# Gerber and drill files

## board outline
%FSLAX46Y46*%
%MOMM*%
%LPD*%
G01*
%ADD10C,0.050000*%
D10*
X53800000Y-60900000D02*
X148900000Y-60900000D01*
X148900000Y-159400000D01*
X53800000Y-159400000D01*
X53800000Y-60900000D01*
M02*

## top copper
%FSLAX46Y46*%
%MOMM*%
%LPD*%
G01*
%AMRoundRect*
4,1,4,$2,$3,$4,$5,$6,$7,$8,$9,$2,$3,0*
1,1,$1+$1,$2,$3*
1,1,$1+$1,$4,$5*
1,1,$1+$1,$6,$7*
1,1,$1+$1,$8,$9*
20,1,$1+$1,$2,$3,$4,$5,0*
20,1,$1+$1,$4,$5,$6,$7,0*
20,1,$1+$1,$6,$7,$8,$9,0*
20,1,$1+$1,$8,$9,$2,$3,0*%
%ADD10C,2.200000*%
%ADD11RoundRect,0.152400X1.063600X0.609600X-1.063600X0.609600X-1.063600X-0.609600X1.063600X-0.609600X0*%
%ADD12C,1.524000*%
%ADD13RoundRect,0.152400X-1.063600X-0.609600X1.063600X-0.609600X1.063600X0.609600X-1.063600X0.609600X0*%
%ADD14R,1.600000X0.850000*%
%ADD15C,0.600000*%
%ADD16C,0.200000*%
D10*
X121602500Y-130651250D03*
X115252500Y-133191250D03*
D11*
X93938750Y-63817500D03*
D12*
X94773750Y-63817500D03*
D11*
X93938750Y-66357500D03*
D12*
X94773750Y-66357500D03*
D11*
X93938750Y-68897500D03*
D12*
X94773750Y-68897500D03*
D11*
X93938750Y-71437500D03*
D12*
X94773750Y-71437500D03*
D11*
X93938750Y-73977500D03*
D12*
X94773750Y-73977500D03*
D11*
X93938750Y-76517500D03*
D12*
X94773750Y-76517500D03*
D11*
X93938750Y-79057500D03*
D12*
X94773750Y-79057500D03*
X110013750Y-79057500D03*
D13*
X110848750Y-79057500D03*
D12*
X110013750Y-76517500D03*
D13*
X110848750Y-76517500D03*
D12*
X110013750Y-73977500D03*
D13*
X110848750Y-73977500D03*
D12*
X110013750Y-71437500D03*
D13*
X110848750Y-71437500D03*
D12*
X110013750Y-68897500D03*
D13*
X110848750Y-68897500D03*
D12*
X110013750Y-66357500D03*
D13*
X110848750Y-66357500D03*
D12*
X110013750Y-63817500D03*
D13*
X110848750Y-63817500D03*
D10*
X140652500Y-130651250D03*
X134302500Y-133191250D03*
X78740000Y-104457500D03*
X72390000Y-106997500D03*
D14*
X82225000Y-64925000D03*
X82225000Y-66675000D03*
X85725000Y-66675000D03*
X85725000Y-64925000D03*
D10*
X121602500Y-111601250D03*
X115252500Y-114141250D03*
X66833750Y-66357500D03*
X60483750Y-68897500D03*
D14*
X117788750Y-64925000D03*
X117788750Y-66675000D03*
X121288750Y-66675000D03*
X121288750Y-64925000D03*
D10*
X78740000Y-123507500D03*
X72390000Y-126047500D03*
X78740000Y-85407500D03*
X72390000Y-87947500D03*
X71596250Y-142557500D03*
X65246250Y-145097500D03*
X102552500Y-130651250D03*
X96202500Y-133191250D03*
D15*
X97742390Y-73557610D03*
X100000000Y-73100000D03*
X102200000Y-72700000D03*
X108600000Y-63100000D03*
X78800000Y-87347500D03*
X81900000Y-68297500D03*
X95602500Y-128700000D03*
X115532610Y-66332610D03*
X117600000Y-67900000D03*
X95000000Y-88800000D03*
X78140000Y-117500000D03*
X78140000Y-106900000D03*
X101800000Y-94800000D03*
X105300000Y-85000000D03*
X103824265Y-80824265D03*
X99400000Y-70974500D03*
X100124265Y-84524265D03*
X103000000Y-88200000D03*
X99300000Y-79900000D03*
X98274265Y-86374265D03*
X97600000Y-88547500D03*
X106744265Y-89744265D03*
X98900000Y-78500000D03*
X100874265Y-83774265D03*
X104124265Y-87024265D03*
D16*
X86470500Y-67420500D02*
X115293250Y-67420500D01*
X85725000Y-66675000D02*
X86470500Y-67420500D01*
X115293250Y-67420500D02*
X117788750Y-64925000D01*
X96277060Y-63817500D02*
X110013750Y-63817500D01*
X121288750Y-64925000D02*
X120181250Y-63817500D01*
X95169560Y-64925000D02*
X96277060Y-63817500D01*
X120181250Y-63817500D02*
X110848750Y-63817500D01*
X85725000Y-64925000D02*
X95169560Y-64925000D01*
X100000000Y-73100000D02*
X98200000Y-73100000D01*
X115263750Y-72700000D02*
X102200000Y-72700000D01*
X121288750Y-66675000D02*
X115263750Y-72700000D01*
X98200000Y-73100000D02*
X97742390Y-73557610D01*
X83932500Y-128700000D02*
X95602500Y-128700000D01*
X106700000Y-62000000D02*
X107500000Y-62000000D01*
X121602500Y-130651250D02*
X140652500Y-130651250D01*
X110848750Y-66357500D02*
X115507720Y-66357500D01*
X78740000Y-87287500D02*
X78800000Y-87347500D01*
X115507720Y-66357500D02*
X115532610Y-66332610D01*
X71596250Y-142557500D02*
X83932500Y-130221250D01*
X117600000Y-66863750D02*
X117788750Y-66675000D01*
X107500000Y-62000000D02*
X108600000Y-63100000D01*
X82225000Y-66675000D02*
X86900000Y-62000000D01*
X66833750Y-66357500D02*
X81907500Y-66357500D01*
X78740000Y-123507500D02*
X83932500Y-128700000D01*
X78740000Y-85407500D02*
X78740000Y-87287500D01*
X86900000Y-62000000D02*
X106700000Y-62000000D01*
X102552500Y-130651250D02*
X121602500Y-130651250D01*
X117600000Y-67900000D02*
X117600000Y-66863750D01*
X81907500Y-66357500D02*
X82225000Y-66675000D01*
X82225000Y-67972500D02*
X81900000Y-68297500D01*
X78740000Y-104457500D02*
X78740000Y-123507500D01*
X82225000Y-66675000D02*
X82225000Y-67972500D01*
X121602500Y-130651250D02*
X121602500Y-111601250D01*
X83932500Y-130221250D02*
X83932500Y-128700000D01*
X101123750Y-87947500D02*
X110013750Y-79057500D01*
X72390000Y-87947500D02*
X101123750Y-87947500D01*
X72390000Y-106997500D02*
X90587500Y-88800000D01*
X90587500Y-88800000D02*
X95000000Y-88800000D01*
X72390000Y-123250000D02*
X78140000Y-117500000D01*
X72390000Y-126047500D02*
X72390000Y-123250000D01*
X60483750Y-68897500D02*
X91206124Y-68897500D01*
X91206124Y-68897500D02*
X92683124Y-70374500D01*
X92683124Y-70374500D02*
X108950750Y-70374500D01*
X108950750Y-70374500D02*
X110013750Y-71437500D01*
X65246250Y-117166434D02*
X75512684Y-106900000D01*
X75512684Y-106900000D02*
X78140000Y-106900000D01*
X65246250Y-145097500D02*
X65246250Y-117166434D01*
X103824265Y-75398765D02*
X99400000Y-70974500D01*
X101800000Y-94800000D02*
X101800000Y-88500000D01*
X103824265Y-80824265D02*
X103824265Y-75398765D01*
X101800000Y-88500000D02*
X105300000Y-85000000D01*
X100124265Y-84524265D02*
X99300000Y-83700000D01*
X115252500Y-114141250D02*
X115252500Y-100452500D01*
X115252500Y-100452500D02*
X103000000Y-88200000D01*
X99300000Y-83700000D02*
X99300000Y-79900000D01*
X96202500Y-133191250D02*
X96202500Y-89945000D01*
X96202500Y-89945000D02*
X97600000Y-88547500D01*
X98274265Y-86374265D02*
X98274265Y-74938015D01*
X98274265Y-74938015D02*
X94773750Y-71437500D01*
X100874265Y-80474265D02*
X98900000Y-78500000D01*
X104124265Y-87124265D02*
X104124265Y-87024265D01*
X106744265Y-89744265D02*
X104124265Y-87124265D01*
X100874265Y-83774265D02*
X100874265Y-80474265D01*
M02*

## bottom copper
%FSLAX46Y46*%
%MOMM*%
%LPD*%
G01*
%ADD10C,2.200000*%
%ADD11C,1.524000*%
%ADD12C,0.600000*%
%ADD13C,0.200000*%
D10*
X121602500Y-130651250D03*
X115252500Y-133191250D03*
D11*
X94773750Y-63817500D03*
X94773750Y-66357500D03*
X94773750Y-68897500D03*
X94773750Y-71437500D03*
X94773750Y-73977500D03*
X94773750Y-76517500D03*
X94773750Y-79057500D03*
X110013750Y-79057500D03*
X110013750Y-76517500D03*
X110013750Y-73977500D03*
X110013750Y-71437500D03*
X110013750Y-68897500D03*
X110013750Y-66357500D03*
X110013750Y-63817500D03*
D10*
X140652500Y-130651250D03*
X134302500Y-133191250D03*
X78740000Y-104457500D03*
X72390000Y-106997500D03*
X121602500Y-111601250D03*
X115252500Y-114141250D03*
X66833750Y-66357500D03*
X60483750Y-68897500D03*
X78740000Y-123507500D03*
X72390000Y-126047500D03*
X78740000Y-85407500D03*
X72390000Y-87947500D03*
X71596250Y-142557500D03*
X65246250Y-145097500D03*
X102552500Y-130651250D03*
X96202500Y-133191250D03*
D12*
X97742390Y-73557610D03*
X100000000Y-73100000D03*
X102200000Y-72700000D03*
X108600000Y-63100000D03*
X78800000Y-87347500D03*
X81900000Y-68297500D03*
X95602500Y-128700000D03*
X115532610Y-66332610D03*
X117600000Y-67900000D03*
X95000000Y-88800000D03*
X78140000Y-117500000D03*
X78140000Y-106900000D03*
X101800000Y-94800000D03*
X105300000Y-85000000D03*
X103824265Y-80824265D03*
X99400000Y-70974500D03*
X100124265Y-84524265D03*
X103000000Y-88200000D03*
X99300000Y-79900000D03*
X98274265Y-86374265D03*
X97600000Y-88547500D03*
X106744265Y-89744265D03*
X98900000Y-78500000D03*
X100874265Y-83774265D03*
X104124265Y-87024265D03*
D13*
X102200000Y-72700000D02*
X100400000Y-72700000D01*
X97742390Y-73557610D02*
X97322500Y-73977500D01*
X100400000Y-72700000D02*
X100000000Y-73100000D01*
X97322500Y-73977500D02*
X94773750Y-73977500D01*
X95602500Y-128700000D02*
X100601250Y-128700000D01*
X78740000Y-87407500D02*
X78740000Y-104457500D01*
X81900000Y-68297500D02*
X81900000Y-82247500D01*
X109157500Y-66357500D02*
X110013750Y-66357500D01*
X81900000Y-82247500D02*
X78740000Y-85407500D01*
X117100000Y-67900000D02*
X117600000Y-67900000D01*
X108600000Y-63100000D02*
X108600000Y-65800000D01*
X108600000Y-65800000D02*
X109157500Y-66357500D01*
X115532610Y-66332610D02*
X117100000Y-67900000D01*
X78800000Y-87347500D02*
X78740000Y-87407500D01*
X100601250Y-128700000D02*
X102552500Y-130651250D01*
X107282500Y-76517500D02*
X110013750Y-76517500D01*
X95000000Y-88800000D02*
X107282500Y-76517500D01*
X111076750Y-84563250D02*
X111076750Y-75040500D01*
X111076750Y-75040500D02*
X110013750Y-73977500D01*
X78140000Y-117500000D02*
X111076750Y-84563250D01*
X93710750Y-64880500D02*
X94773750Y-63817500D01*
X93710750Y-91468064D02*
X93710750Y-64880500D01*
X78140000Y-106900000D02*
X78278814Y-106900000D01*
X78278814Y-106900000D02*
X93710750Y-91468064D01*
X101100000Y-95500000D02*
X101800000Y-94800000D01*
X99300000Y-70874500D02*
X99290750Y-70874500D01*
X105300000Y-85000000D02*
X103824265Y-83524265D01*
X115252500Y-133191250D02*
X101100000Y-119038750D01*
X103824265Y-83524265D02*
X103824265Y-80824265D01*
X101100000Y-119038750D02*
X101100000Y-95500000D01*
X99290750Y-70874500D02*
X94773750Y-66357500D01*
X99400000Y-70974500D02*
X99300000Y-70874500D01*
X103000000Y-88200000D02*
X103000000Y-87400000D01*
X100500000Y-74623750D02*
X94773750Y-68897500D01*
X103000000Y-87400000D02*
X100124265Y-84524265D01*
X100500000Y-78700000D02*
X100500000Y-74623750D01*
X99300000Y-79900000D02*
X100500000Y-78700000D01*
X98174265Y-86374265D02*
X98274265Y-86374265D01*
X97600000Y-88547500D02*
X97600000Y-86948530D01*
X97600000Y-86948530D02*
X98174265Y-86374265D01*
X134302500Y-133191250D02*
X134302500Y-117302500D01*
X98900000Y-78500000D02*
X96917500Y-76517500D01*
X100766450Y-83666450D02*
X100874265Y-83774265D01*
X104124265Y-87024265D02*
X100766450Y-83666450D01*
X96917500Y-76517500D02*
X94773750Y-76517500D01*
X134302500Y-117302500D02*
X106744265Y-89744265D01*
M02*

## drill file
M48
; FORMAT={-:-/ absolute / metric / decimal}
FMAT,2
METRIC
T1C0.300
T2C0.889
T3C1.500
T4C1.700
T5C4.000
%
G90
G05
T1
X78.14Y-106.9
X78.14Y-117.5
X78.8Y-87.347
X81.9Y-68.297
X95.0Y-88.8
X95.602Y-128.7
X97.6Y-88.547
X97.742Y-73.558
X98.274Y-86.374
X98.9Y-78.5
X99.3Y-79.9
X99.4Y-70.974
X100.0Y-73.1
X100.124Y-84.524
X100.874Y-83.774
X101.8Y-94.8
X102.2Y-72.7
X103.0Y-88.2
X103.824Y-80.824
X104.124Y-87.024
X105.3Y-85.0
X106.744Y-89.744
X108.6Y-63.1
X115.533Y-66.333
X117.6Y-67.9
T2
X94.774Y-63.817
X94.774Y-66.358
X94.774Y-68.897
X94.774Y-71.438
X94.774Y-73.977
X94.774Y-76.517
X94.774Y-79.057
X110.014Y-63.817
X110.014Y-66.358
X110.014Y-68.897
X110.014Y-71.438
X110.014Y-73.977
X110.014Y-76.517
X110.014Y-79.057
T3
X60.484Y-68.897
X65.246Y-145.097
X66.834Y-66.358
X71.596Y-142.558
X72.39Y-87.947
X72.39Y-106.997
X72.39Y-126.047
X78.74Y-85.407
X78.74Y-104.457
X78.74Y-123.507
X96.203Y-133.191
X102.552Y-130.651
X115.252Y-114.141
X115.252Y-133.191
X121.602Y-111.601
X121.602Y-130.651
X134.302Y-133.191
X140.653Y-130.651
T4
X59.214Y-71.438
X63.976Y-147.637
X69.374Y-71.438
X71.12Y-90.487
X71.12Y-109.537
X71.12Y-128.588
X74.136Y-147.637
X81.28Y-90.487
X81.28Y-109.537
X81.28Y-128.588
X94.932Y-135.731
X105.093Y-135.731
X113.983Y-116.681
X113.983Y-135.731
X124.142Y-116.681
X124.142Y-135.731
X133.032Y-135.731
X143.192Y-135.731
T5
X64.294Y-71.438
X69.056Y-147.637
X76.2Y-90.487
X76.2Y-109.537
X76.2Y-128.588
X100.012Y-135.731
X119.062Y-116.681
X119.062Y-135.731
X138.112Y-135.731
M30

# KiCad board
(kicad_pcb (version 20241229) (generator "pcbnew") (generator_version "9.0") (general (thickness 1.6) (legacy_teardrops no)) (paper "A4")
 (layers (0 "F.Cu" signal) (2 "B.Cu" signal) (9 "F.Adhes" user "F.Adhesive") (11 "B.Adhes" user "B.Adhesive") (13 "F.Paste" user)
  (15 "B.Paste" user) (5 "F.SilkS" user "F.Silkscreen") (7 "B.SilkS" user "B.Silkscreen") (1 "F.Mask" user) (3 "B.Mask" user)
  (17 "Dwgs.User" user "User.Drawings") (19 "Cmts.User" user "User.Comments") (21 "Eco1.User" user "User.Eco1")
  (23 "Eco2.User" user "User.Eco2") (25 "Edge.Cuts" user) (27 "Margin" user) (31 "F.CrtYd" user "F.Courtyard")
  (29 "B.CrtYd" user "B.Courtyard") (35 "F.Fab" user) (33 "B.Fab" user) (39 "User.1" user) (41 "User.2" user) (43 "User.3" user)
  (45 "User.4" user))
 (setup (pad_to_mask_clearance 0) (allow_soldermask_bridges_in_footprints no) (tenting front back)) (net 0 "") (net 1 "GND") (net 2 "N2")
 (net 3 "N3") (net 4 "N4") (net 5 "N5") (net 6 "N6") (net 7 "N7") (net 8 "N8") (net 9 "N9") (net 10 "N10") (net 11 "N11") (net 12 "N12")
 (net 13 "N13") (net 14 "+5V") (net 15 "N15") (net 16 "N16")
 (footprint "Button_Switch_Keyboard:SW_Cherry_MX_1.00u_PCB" (layer "F.Cu") (at 121.6025 130.65125)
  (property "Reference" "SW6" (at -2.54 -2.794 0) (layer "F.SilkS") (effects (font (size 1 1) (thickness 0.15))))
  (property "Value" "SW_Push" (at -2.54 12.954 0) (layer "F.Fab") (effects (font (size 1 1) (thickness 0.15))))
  (pad "" np_thru_hole circle (at -7.62 5.08) (size 1.7 1.7) (drill 1.7) (layers "*.Cu" "*.Mask"))
  (pad "" np_thru_hole circle (at -2.54 5.08) (size 4 4) (drill 4) (layers "*.Cu" "*.Mask"))
  (pad "" np_thru_hole circle (at 2.54 5.08) (size 1.7 1.7) (drill 1.7) (layers "*.Cu" "*.Mask"))
  (pad "1" thru_hole circle (at 0 0) (size 2.2 2.2) (drill 1.5) (layers "*.Cu" "*.Mask") (remove_unused_layers no) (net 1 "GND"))
  (pad "2" thru_hole circle (at -6.35 2.54) (size 2.2 2.2) (drill 1.5) (layers "*.Cu" "*.Mask") (remove_unused_layers no) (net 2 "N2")))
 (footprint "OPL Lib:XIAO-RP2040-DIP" (layer "F.Cu") (at 102.39375 71.4375)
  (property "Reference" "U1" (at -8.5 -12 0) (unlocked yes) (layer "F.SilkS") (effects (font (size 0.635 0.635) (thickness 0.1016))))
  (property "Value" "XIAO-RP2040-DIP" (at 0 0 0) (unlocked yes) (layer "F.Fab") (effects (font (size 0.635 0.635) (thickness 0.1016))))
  (pad "1" smd roundrect (at -8.455 -7.62 180) (size 2.432 1.524) (layers "F.Cu" "F.Mask") (roundrect_rratio 0.1) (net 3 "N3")
   (thermal_bridge_angle 45))
  (pad "1" thru_hole circle (at -7.62 -7.62 180) (size 1.524 1.524) (drill 0.889) (layers "*.Cu" "*.Mask") (remove_unused_layers no)
   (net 3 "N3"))
  (pad "2" smd roundrect (at -8.455 -5.08 180) (size 2.432 1.524) (layers "F.Cu" "F.Mask") (roundrect_rratio 0.1) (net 2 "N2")
   (thermal_bridge_angle 45))
  (pad "2" thru_hole circle (at -7.62 -5.08 180) (size 1.524 1.524) (drill 0.889) (layers "*.Cu" "*.Mask") (remove_unused_layers no)
   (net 2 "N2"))
  (pad "3" smd roundrect (at -8.455 -2.54 180) (size 2.432 1.524) (layers "F.Cu" "F.Mask") (roundrect_rratio 0.1) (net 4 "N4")
   (thermal_bridge_angle 45))
  (pad "3" thru_hole circle (at -7.62 -2.54 180) (size 1.524 1.524) (drill 0.889) (layers "*.Cu" "*.Mask") (remove_unused_layers no)
   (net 4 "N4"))
  (pad "4" smd roundrect (at -8.455 0 180) (size 2.432 1.524) (layers "F.Cu" "F.Mask") (roundrect_rratio 0.1) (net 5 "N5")
   (thermal_bridge_angle 45))
  (pad "4" thru_hole circle (at -7.62 0 180) (size 1.524 1.524) (drill 0.889) (layers "*.Cu" "*.Mask") (remove_unused_layers no)
   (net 5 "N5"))
  (pad "5" smd roundrect (at -8.455 2.54 180) (size 2.432 1.524) (layers "F.Cu" "F.Mask") (roundrect_rratio 0.1) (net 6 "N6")
   (thermal_bridge_angle 45))
  (pad "5" thru_hole circle (at -7.62 2.54 180) (size 1.524 1.524) (drill 0.889) (layers "*.Cu" "*.Mask") (remove_unused_layers no)
   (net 6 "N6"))
  (pad "6" smd roundrect (at -8.455 5.08 180) (size 2.432 1.524) (layers "F.Cu" "F.Mask") (roundrect_rratio 0.1) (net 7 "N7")
   (thermal_bridge_angle 45))
  (pad "6" thru_hole circle (at -7.62 5.08 180) (size 1.524 1.524) (drill 0.889) (layers "*.Cu" "*.Mask") (remove_unused_layers no)
   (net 7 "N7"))
  (pad "7" smd roundrect (at -8.455 7.62 180) (size 2.432 1.524) (layers "F.Cu" "F.Mask") (roundrect_rratio 0.1) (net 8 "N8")
   (thermal_bridge_angle 45))
  (pad "7" thru_hole circle (at -7.62 7.62 180) (size 1.524 1.524) (drill 0.889) (layers "*.Cu" "*.Mask") (remove_unused_layers no)
   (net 8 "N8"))
  (pad "8" thru_hole circle (at 7.62 7.62) (size 1.524 1.524) (drill 0.889) (layers "*.Cu" "*.Mask") (remove_unused_layers no) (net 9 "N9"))
  (pad "8" smd roundrect (at 8.455 7.62) (size 2.432 1.524) (layers "F.Cu" "F.Mask") (roundrect_rratio 0.1) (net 9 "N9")
   (thermal_bridge_angle 45))
  (pad "9" thru_hole circle (at 7.62 5.08) (size 1.524 1.524) (drill 0.889) (layers "*.Cu" "*.Mask") (remove_unused_layers no)
   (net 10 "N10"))
  (pad "9" smd roundrect (at 8.455 5.08) (size 2.432 1.524) (layers "F.Cu" "F.Mask") (roundrect_rratio 0.1) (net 10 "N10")
   (thermal_bridge_angle 45))
  (pad "10" thru_hole circle (at 7.62 2.54) (size 1.524 1.524) (drill 0.889) (layers "*.Cu" "*.Mask") (remove_unused_layers no)
   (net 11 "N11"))
  (pad "10" smd roundrect (at 8.455 2.54) (size 2.432 1.524) (layers "F.Cu" "F.Mask") (roundrect_rratio 0.1) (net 11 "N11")
   (thermal_bridge_angle 45))
  (pad "11" thru_hole circle (at 7.62 0) (size 1.524 1.524) (drill 0.889) (layers "*.Cu" "*.Mask") (remove_unused_layers no) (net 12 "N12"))
  (pad "11" smd roundrect (at 8.455 0) (size 2.432 1.524) (layers "F.Cu" "F.Mask") (roundrect_rratio 0.1) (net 12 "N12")
   (thermal_bridge_angle 45))
  (pad "12" thru_hole circle (at 7.62 -2.54) (size 1.524 1.524) (drill 0.889) (layers "*.Cu" "*.Mask") (remove_unused_layers no)
   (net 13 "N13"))
  (pad "12" smd roundrect (at 8.455 -2.54) (size 2.432 1.524) (layers "F.Cu" "F.Mask") (roundrect_rratio 0.1) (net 13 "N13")
   (thermal_bridge_angle 45))
  (pad "13" thru_hole circle (at 7.62 -5.08) (size 1.524 1.524) (drill 0.889) (layers "*.Cu" "*.Mask") (remove_unused_layers no)
   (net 1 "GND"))
  (pad "13" smd roundrect (at 8.455 -5.08) (size 2.432 1.524) (layers "F.Cu" "F.Mask") (roundrect_rratio 0.1) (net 1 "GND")
   (thermal_bridge_angle 45))
  (pad "14" thru_hole circle (at 7.62 -7.62) (size 1.524 1.524) (drill 0.889) (layers "*.Cu" "*.Mask") (remove_unused_layers no)
   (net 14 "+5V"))
  (pad "14" smd roundrect (at 8.455 -7.62) (size 2.432 1.524) (layers "F.Cu" "F.Mask") (roundrect_rratio 0.1) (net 14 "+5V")
   (thermal_bridge_angle 45)))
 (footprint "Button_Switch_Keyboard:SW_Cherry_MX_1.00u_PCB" (layer "F.Cu") (at 140.6525 130.65125)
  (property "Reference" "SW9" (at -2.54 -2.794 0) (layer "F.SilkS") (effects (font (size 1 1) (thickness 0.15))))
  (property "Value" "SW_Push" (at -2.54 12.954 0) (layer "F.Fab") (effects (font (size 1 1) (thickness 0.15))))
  (pad "" np_thru_hole circle (at -7.62 5.08) (size 1.7 1.7) (drill 1.7) (layers "*.Cu" "*.Mask"))
  (pad "" np_thru_hole circle (at -2.54 5.08) (size 4 4) (drill 4) (layers "*.Cu" "*.Mask"))
  (pad "" np_thru_hole circle (at 2.54 5.08) (size 1.7 1.7) (drill 1.7) (layers "*.Cu" "*.Mask"))
  (pad "1" thru_hole circle (at 0 0) (size 2.2 2.2) (drill 1.5) (layers "*.Cu" "*.Mask") (remove_unused_layers no) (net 1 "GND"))
  (pad "2" thru_hole circle (at -6.35 2.54) (size 2.2 2.2) (drill 1.5) (layers "*.Cu" "*.Mask") (remove_unused_layers no) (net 7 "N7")))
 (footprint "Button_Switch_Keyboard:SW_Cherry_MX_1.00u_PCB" (layer "F.Cu") (at 78.74 104.4575)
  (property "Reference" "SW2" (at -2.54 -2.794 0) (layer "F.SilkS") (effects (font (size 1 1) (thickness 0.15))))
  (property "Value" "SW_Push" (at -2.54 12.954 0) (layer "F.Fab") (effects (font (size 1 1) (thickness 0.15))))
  (pad "" np_thru_hole circle (at -7.62 5.08) (size 1.7 1.7) (drill 1.7) (layers "*.Cu" "*.Mask"))
  (pad "" np_thru_hole circle (at -2.54 5.08) (size 4 4) (drill 4) (layers "*.Cu" "*.Mask"))
  (pad "" np_thru_hole circle (at 2.54 5.08) (size 1.7 1.7) (drill 1.7) (layers "*.Cu" "*.Mask"))
  (pad "1" thru_hole circle (at 0 0) (size 2.2 2.2) (drill 1.5) (layers "*.Cu" "*.Mask") (remove_unused_layers no) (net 1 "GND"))
  (pad "2" thru_hole circle (at -6.35 2.54) (size 2.2 2.2) (drill 1.5) (layers "*.Cu" "*.Mask") (remove_unused_layers no) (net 10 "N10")))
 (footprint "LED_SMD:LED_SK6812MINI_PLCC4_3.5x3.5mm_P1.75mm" (layer "F.Cu") (at 83.975 65.8)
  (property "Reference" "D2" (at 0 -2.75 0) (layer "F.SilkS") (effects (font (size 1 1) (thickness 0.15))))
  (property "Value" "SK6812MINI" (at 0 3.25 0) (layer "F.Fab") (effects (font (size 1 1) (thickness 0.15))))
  (pad "1" smd rect (at -1.75 -0.875) (size 1.6 0.85) (layers "F.Cu" "F.Mask" "F.Paste") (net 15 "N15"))
  (pad "2" smd rect (at -1.75 0.875) (size 1.6 0.85) (layers "F.Cu" "F.Mask" "F.Paste") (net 1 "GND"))
  (pad "3" smd rect (at 1.75 0.875) (size 1.6 0.85) (layers "F.Cu" "F.Mask" "F.Paste") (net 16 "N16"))
  (pad "4" smd rect (at 1.75 -0.875) (size 1.6 0.85) (layers "F.Cu" "F.Mask" "F.Paste") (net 14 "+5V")))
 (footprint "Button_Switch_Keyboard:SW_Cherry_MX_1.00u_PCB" (layer "F.Cu") (at 121.6025 111.60125)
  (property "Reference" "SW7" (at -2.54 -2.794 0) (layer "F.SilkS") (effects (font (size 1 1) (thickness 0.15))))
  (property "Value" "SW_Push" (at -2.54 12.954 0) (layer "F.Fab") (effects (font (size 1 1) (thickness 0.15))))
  (pad "" np_thru_hole circle (at -7.62 5.08) (size 1.7 1.7) (drill 1.7) (layers "*.Cu" "*.Mask"))
  (pad "" np_thru_hole circle (at -2.54 5.08) (size 4 4) (drill 4) (layers "*.Cu" "*.Mask"))
  (pad "" np_thru_hole circle (at 2.54 5.08) (size 1.7 1.7) (drill 1.7) (layers "*.Cu" "*.Mask"))
  (pad "1" thru_hole circle (at 0 0) (size 2.2 2.2) (drill 1.5) (layers "*.Cu" "*.Mask") (remove_unused_layers no) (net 1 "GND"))
  (pad "2" thru_hole circle (at -6.35 2.54) (size 2.2 2.2) (drill 1.5) (layers "*.Cu" "*.Mask") (remove_unused_layers no) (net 4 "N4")))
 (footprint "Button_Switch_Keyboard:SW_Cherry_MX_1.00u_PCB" (layer "F.Cu") (at 66.83375 66.3575)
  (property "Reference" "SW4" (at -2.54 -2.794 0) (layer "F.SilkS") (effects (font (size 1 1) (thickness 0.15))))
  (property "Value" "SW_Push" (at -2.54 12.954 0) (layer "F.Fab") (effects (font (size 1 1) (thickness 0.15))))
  (pad "" np_thru_hole circle (at -7.62 5.08) (size 1.7 1.7) (drill 1.7) (layers "*.Cu" "*.Mask"))
  (pad "" np_thru_hole circle (at -2.54 5.08) (size 4 4) (drill 4) (layers "*.Cu" "*.Mask"))
  (pad "" np_thru_hole circle (at 2.54 5.08) (size 1.7 1.7) (drill 1.7) (layers "*.Cu" "*.Mask"))
  (pad "1" thru_hole circle (at 0 0) (size 2.2 2.2) (drill 1.5) (layers "*.Cu" "*.Mask") (remove_unused_layers no) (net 1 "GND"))
  (pad "2" thru_hole circle (at -6.35 2.54) (size 2.2 2.2) (drill 1.5) (layers "*.Cu" "*.Mask") (remove_unused_layers no) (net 12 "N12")))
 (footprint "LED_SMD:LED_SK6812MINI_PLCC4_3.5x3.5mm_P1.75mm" (layer "F.Cu") (at 119.53875 65.8)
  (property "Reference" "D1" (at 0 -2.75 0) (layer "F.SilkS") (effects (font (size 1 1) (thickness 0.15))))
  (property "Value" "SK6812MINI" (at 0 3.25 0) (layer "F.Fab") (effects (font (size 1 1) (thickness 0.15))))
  (pad "1" smd rect (at -1.75 -0.875) (size 1.6 0.85) (layers "F.Cu" "F.Mask" "F.Paste") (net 16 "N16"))
  (pad "2" smd rect (at -1.75 0.875) (size 1.6 0.85) (layers "F.Cu" "F.Mask" "F.Paste") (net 1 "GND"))
  (pad "3" smd rect (at 1.75 0.875) (size 1.6 0.85) (layers "F.Cu" "F.Mask" "F.Paste") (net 6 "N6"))
  (pad "4" smd rect (at 1.75 -0.875) (size 1.6 0.85) (layers "F.Cu" "F.Mask" "F.Paste") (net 14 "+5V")))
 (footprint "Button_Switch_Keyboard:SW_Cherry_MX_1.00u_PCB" (layer "F.Cu") (at 78.74 123.5075)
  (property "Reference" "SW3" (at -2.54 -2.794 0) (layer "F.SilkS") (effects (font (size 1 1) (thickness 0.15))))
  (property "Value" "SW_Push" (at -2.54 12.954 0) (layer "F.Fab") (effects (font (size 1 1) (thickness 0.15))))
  (pad "" np_thru_hole circle (at -7.62 5.08) (size 1.7 1.7) (drill 1.7) (layers "*.Cu" "*.Mask"))
  (pad "" np_thru_hole circle (at -2.54 5.08) (size 4 4) (drill 4) (layers "*.Cu" "*.Mask"))
  (pad "" np_thru_hole circle (at 2.54 5.08) (size 1.7 1.7) (drill 1.7) (layers "*.Cu" "*.Mask"))
  (pad "1" thru_hole circle (at 0 0) (size 2.2 2.2) (drill 1.5) (layers "*.Cu" "*.Mask") (remove_unused_layers no) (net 1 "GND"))
  (pad "2" thru_hole circle (at -6.35 2.54) (size 2.2 2.2) (drill 1.5) (layers "*.Cu" "*.Mask") (remove_unused_layers no) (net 11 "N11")))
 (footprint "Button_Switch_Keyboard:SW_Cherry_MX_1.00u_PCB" (layer "F.Cu") (at 78.74 85.4075)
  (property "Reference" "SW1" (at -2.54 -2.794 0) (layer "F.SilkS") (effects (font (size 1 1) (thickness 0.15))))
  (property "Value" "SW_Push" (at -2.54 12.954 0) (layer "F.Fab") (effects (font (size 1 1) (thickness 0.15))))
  (pad "" np_thru_hole circle (at -7.62 5.08) (size 1.7 1.7) (drill 1.7) (layers "*.Cu" "*.Mask"))
  (pad "" np_thru_hole circle (at -2.54 5.08) (size 4 4) (drill 4) (layers "*.Cu" "*.Mask"))
  (pad "" np_thru_hole circle (at 2.54 5.08) (size 1.7 1.7) (drill 1.7) (layers "*.Cu" "*.Mask"))
  (pad "1" thru_hole circle (at 0 0) (size 2.2 2.2) (drill 1.5) (layers "*.Cu" "*.Mask") (remove_unused_layers no) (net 1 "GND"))
  (pad "2" thru_hole circle (at -6.35 2.54) (size 2.2 2.2) (drill 1.5) (layers "*.Cu" "*.Mask") (remove_unused_layers no) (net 9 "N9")))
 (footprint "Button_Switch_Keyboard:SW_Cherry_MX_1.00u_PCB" (layer "F.Cu") (at 71.59625 142.5575)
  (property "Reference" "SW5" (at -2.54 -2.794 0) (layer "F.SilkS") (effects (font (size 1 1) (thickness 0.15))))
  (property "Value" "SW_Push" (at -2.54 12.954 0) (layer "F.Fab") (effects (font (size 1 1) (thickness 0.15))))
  (pad "" np_thru_hole circle (at -7.62 5.08) (size 1.7 1.7) (drill 1.7) (layers "*.Cu" "*.Mask"))
  (pad "" np_thru_hole circle (at -2.54 5.08) (size 4 4) (drill 4) (layers "*.Cu" "*.Mask"))
  (pad "" np_thru_hole circle (at 2.54 5.08) (size 1.7 1.7) (drill 1.7) (layers "*.Cu" "*.Mask"))
  (pad "1" thru_hole circle (at 0 0) (size 2.2 2.2) (drill 1.5) (layers "*.Cu" "*.Mask") (remove_unused_layers no) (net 1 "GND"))
  (pad "2" thru_hole circle (at -6.35 2.54) (size 2.2 2.2) (drill 1.5) (layers "*.Cu" "*.Mask") (remove_unused_layers no) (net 3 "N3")))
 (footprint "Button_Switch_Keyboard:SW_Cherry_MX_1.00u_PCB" (layer "F.Cu") (at 102.5525 130.65125)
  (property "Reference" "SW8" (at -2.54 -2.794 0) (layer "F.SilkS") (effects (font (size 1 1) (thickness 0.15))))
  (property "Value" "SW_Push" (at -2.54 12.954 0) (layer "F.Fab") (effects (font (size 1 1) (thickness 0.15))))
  (pad "" np_thru_hole circle (at -7.62 5.08) (size 1.7 1.7) (drill 1.7) (layers "*.Cu" "*.Mask"))
  (pad "" np_thru_hole circle (at -2.54 5.08) (size 4 4) (drill 4) (layers "*.Cu" "*.Mask"))
  (pad "" np_thru_hole circle (at 2.54 5.08) (size 1.7 1.7) (drill 1.7) (layers "*.Cu" "*.Mask"))
  (pad "1" thru_hole circle (at 0 0) (size 2.2 2.2) (drill 1.5) (layers "*.Cu" "*.Mask") (remove_unused_layers no) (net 1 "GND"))
  (pad "2" thru_hole circle (at -6.35 2.54) (size 2.2 2.2) (drill 1.5) (layers "*.Cu" "*.Mask") (remove_unused_layers no) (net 5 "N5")))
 (gr_rect (start 53.8 60.9) (end 148.9 159.4) (stroke (width 0.05) (type default)) (fill no) (layer "Edge.Cuts"))
 (segment (start 86.4705 67.4205) (end 115.29325 67.4205) (width 0.2) (layer "F.Cu") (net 16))
 (segment (start 85.725 66.675) (end 86.4705 67.4205) (width 0.2) (layer "F.Cu") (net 16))
 (segment (start 115.29325 67.4205) (end 117.78875 64.925) (width 0.2) (layer "F.Cu") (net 16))
 (segment (start 96.27706 63.8175) (end 110.01375 63.8175) (width 0.2) (layer "F.Cu") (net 14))
 (segment (start 121.28875 64.925) (end 120.18125 63.8175) (width 0.2) (layer "F.Cu") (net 14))
 (segment (start 95.16956 64.925) (end 96.27706 63.8175) (width 0.2) (layer "F.Cu") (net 14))
 (segment (start 120.18125 63.8175) (end 110.84875 63.8175) (width 0.2) (layer "F.Cu") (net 14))
 (segment (start 85.725 64.925) (end 95.16956 64.925) (width 0.2) (layer "F.Cu") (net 14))
 (segment (start 100 73.1) (end 98.2 73.1) (width 0.2) (layer "F.Cu") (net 6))
 (segment (start 115.26375 72.7) (end 102.2 72.7) (width 0.2) (layer "F.Cu") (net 6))
 (segment (start 121.28875 66.675) (end 115.26375 72.7) (width 0.2) (layer "F.Cu") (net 6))
 (segment (start 98.2 73.1) (end 97.74239 73.55761) (width 0.2) (layer "F.Cu") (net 6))
 (via (at 97.74239 73.55761) (size 0.6) (drill 0.3) (layers "F.Cu" "B.Cu") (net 6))
 (via (at 100 73.1) (size 0.6) (drill 0.3) (layers "F.Cu" "B.Cu") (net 6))
 (via (at 102.2 72.7) (size 0.6) (drill 0.3) (layers "F.Cu" "B.Cu") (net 6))
 (segment (start 102.2 72.7) (end 100.4 72.7) (width 0.2) (layer "B.Cu") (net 6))
 (segment (start 97.74239 73.55761) (end 97.3225 73.9775) (width 0.2) (layer "B.Cu") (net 6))
 (segment (start 100.4 72.7) (end 100 73.1) (width 0.2) (layer "B.Cu") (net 6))
 (segment (start 97.3225 73.9775) (end 94.77375 73.9775) (width 0.2) (layer "B.Cu") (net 6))
 (segment (start 83.9325 128.7) (end 95.6025 128.7) (width 0.2) (layer "F.Cu") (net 1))
 (segment (start 106.7 62) (end 107.5 62) (width 0.2) (layer "F.Cu") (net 1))
 (segment (start 121.6025 130.65125) (end 140.6525 130.65125) (width 0.2) (layer "F.Cu") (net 1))
 (segment (start 110.84875 66.3575) (end 115.50772 66.3575) (width 0.2) (layer "F.Cu") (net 1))
 (segment (start 78.74 87.2875) (end 78.8 87.3475) (width 0.2) (layer "F.Cu") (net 1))
 (segment (start 115.50772 66.3575) (end 115.53261 66.33261) (width 0.2) (layer "F.Cu") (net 1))
 (segment (start 71.59625 142.5575) (end 83.9325 130.22125) (width 0.2) (layer "F.Cu") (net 1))
 (segment (start 117.6 66.86375) (end 117.78875 66.675) (width 0.2) (layer "F.Cu") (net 1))
 (segment (start 107.5 62) (end 108.6 63.1) (width 0.2) (layer "F.Cu") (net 1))
 (segment (start 82.225 66.675) (end 86.9 62) (width 0.2) (layer "F.Cu") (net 1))
 (segment (start 66.83375 66.3575) (end 81.9075 66.3575) (width 0.2) (layer "F.Cu") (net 1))
 (segment (start 78.74 123.5075) (end 83.9325 128.7) (width 0.2) (layer "F.Cu") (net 1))
 (segment (start 78.74 85.4075) (end 78.74 87.2875) (width 0.2) (layer "F.Cu") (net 1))
 (segment (start 86.9 62) (end 106.7 62) (width 0.2) (layer "F.Cu") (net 1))
 (segment (start 102.5525 130.65125) (end 121.6025 130.65125) (width 0.2) (layer "F.Cu") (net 1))
 (segment (start 117.6 67.9) (end 117.6 66.86375) (width 0.2) (layer "F.Cu") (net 1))
 (segment (start 81.9075 66.3575) (end 82.225 66.675) (width 0.2) (layer "F.Cu") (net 1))
 (segment (start 82.225 67.9725) (end 81.9 68.2975) (width 0.2) (layer "F.Cu") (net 1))
 (segment (start 78.74 104.4575) (end 78.74 123.5075) (width 0.2) (layer "F.Cu") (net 1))
 (segment (start 82.225 66.675) (end 82.225 67.9725) (width 0.2) (layer "F.Cu") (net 1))
 (segment (start 121.6025 130.65125) (end 121.6025 111.60125) (width 0.2) (layer "F.Cu") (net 1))
 (segment (start 83.9325 130.22125) (end 83.9325 128.7) (width 0.2) (layer "F.Cu") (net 1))
 (via (at 108.6 63.1) (size 0.6) (drill 0.3) (layers "F.Cu" "B.Cu") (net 1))
 (via (at 78.8 87.3475) (size 0.6) (drill 0.3) (layers "F.Cu" "B.Cu") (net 1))
 (via (at 81.9 68.2975) (size 0.6) (drill 0.3) (layers "F.Cu" "B.Cu") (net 1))
 (via (at 95.6025 128.7) (size 0.6) (drill 0.3) (layers "F.Cu" "B.Cu") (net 1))
 (via (at 115.53261 66.33261) (size 0.6) (drill 0.3) (layers "F.Cu" "B.Cu") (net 1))
 (via (at 117.6 67.9) (size 0.6) (drill 0.3) (layers "F.Cu" "B.Cu") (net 1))
 (segment (start 95.6025 128.7) (end 100.60125 128.7) (width 0.2) (layer "B.Cu") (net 1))
 (segment (start 78.74 87.4075) (end 78.74 104.4575) (width 0.2) (layer "B.Cu") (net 1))
 (segment (start 81.9 68.2975) (end 81.9 82.2475) (width 0.2) (layer "B.Cu") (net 1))
 (segment (start 109.1575 66.3575) (end 110.01375 66.3575) (width 0.2) (layer "B.Cu") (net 1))
 (segment (start 81.9 82.2475) (end 78.74 85.4075) (width 0.2) (layer "B.Cu") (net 1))
 (segment (start 117.1 67.9) (end 117.6 67.9) (width 0.2) (layer "B.Cu") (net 1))
 (segment (start 108.6 63.1) (end 108.6 65.8) (width 0.2) (layer "B.Cu") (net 1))
 (segment (start 108.6 65.8) (end 109.1575 66.3575) (width 0.2) (layer "B.Cu") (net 1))
 (segment (start 115.53261 66.33261) (end 117.1 67.9) (width 0.2) (layer "B.Cu") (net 1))
 (segment (start 78.8 87.3475) (end 78.74 87.4075) (width 0.2) (layer "B.Cu") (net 1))
 (segment (start 100.60125 128.7) (end 102.5525 130.65125) (width 0.2) (layer "B.Cu") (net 1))
 (segment (start 101.12375 87.9475) (end 110.01375 79.0575) (width 0.2) (layer "F.Cu") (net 9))
 (segment (start 72.39 87.9475) (end 101.12375 87.9475) (width 0.2) (layer "F.Cu") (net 9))
 (segment (start 72.39 106.9975) (end 90.5875 88.8) (width 0.2) (layer "F.Cu") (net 10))
 (segment (start 90.5875 88.8) (end 95 88.8) (width 0.2) (layer "F.Cu") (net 10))
 (via (at 95 88.8) (size 0.6) (drill 0.3) (layers "F.Cu" "B.Cu") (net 10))
 (segment (start 107.2825 76.5175) (end 110.01375 76.5175) (width 0.2) (layer "B.Cu") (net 10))
 (segment (start 95 88.8) (end 107.2825 76.5175) (width 0.2) (layer "B.Cu") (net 10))
 (segment (start 72.39 123.25) (end 78.14 117.5) (width 0.2) (layer "F.Cu") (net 11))
 (segment (start 72.39 126.0475) (end 72.39 123.25) (width 0.2) (layer "F.Cu") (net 11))
 (via (at 78.14 117.5) (size 0.6) (drill 0.3) (layers "F.Cu" "B.Cu") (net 11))
 (segment (start 111.07675 84.56325) (end 111.07675 75.0405) (width 0.2) (layer "B.Cu") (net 11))
 (segment (start 111.07675 75.0405) (end 110.01375 73.9775) (width 0.2) (layer "B.Cu") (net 11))
 (segment (start 78.14 117.5) (end 111.07675 84.56325) (width 0.2) (layer "B.Cu") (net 11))
 (segment (start 60.48375 68.8975) (end 91.206124 68.8975) (width 0.2) (layer "F.Cu") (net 12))
 (segment (start 91.206124 68.8975) (end 92.683124 70.3745) (width 0.2) (layer "F.Cu") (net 12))
 (segment (start 92.683124 70.3745) (end 108.95075 70.3745) (width 0.2) (layer "F.Cu") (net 12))
 (segment (start 108.95075 70.3745) (end 110.01375 71.4375) (width 0.2) (layer "F.Cu") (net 12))
 (segment (start 65.24625 117.166434) (end 75.512684 106.9) (width 0.2) (layer "F.Cu") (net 3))
 (segment (start 75.512684 106.9) (end 78.14 106.9) (width 0.2) (layer "F.Cu") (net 3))
 (segment (start 65.24625 145.0975) (end 65.24625 117.166434) (width 0.2) (layer "F.Cu") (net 3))
 (via (at 78.14 106.9) (size 0.6) (drill 0.3) (layers "F.Cu" "B.Cu") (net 3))
 (segment (start 93.71075 64.8805) (end 94.77375 63.8175) (width 0.2) (layer "B.Cu") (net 3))
 (segment (start 93.71075 91.468064) (end 93.71075 64.8805) (width 0.2) (layer "B.Cu") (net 3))
 (segment (start 78.14 106.9) (end 78.278814 106.9) (width 0.2) (layer "B.Cu") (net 3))
 (segment (start 78.278814 106.9) (end 93.71075 91.468064) (width 0.2) (layer "B.Cu") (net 3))
 (segment (start 103.824265 75.398765) (end 99.4 70.9745) (width 0.2) (layer "F.Cu") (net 2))
 (segment (start 101.8 94.8) (end 101.8 88.5) (width 0.2) (layer "F.Cu") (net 2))
 (segment (start 103.824265 80.824265) (end 103.824265 75.398765) (width 0.2) (layer "F.Cu") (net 2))
 (segment (start 101.8 88.5) (end 105.3 85) (width 0.2) (layer "F.Cu") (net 2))
 (via (at 101.8 94.8) (size 0.6) (drill 0.3) (layers "F.Cu" "B.Cu") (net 2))
 (via (at 105.3 85) (size 0.6) (drill 0.3) (layers "F.Cu" "B.Cu") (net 2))
 (via (at 103.824265 80.824265) (size 0.6) (drill 0.3) (layers "F.Cu" "B.Cu") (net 2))
 (via (at 99.4 70.9745) (size 0.6) (drill 0.3) (layers "F.Cu" "B.Cu") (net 2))
 (segment (start 101.1 95.5) (end 101.8 94.8) (width 0.2) (layer "B.Cu") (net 2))
 (segment (start 99.3 70.8745) (end 99.29075 70.8745) (width 0.2) (layer "B.Cu") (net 2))
 (segment (start 105.3 85) (end 103.824265 83.524265) (width 0.2) (layer "B.Cu") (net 2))
 (segment (start 115.2525 133.19125) (end 101.1 119.03875) (width 0.2) (layer "B.Cu") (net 2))
 (segment (start 103.824265 83.524265) (end 103.824265 80.824265) (width 0.2) (layer "B.Cu") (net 2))
 (segment (start 101.1 119.03875) (end 101.1 95.5) (width 0.2) (layer "B.Cu") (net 2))
 (segment (start 99.29075 70.8745) (end 94.77375 66.3575) (width 0.2) (layer "B.Cu") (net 2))
 (segment (start 99.4 70.9745) (end 99.3 70.8745) (width 0.2) (layer "B.Cu") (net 2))
 (segment (start 100.124265 84.524265) (end 99.3 83.7) (width 0.2) (layer "F.Cu") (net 4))
 (segment (start 115.2525 114.14125) (end 115.2525 100.4525) (width 0.2) (layer "F.Cu") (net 4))
 (segment (start 115.2525 100.4525) (end 103 88.2) (width 0.2) (layer "F.Cu") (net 4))
 (segment (start 99.3 83.7) (end 99.3 79.9) (width 0.2) (layer "F.Cu") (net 4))
 (via (at 100.124265 84.524265) (size 0.6) (drill 0.3) (layers "F.Cu" "B.Cu") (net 4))
 (via (at 103 88.2) (size 0.6) (drill 0.3) (layers "F.Cu" "B.Cu") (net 4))
 (via (at 99.3 79.9) (size 0.6) (drill 0.3) (layers "F.Cu" "B.Cu") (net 4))
 (segment (start 103 88.2) (end 103 87.4) (width 0.2) (layer "B.Cu") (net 4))
 (segment (start 100.5 74.62375) (end 94.77375 68.8975) (width 0.2) (layer "B.Cu") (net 4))
 (segment (start 103 87.4) (end 100.124265 84.524265) (width 0.2) (layer "B.Cu") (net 4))
 (segment (start 100.5 78.7) (end 100.5 74.62375) (width 0.2) (layer "B.Cu") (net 4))
 (segment (start 99.3 79.9) (end 100.5 78.7) (width 0.2) (layer "B.Cu") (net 4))
 (segment (start 96.2025 133.19125) (end 96.2025 89.945) (width 0.2) (layer "F.Cu") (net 5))
 (segment (start 96.2025 89.945) (end 97.6 88.5475) (width 0.2) (layer "F.Cu") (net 5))
 (segment (start 98.274265 86.374265) (end 98.274265 74.938015) (width 0.2) (layer "F.Cu") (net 5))
 (segment (start 98.274265 74.938015) (end 94.77375 71.4375) (width 0.2) (layer "F.Cu") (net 5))
 (via (at 98.274265 86.374265) (size 0.6) (drill 0.3) (layers "F.Cu" "B.Cu") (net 5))
 (via (at 97.6 88.5475) (size 0.6) (drill 0.3) (layers "F.Cu" "B.Cu") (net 5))
 (segment (start 98.174265 86.374265) (end 98.274265 86.374265) (width 0.2) (layer "B.Cu") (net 5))
 (segment (start 97.6 88.5475) (end 97.6 86.94853) (width 0.2) (layer "B.Cu") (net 5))
 (segment (start 97.6 86.94853) (end 98.174265 86.374265) (width 0.2) (layer "B.Cu") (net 5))
 (segment (start 100.874265 80.474265) (end 98.9 78.5) (width 0.2) (layer "F.Cu") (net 7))
 (segment (start 104.124265 87.124265) (end 104.124265 87.024265) (width 0.2) (layer "F.Cu") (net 7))
 (segment (start 106.744265 89.744265) (end 104.124265 87.124265) (width 0.2) (layer "F.Cu") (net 7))
 (segment (start 100.874265 83.774265) (end 100.874265 80.474265) (width 0.2) (layer "F.Cu") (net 7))
 (via (at 106.744265 89.744265) (size 0.6) (drill 0.3) (layers "F.Cu" "B.Cu") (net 7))
 (via (at 98.9 78.5) (size 0.6) (drill 0.3) (layers "F.Cu" "B.Cu") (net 7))
 (via (at 100.874265 83.774265) (size 0.6) (drill 0.3) (layers "F.Cu" "B.Cu") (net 7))
 (via (at 104.124265 87.024265) (size 0.6) (drill 0.3) (layers "F.Cu" "B.Cu") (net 7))
 (segment (start 134.3025 133.19125) (end 134.3025 117.3025) (width 0.2) (layer "B.Cu") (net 7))
 (segment (start 98.9 78.5) (end 96.9175 76.5175) (width 0.2) (layer "B.Cu") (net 7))
 (segment (start 100.76645 83.66645) (end 100.874265 83.774265) (width 0.2) (layer "B.Cu") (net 7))
 (segment (start 104.124265 87.024265) (end 100.76645 83.66645) (width 0.2) (layer "B.Cu") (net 7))
 (segment (start 96.9175 76.5175) (end 94.77375 76.5175) (width 0.2) (layer "B.Cu") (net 7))
 (segment (start 134.3025 117.3025) (end 106.744265 89.744265) (width 0.2) (layer "B.Cu") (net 7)))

